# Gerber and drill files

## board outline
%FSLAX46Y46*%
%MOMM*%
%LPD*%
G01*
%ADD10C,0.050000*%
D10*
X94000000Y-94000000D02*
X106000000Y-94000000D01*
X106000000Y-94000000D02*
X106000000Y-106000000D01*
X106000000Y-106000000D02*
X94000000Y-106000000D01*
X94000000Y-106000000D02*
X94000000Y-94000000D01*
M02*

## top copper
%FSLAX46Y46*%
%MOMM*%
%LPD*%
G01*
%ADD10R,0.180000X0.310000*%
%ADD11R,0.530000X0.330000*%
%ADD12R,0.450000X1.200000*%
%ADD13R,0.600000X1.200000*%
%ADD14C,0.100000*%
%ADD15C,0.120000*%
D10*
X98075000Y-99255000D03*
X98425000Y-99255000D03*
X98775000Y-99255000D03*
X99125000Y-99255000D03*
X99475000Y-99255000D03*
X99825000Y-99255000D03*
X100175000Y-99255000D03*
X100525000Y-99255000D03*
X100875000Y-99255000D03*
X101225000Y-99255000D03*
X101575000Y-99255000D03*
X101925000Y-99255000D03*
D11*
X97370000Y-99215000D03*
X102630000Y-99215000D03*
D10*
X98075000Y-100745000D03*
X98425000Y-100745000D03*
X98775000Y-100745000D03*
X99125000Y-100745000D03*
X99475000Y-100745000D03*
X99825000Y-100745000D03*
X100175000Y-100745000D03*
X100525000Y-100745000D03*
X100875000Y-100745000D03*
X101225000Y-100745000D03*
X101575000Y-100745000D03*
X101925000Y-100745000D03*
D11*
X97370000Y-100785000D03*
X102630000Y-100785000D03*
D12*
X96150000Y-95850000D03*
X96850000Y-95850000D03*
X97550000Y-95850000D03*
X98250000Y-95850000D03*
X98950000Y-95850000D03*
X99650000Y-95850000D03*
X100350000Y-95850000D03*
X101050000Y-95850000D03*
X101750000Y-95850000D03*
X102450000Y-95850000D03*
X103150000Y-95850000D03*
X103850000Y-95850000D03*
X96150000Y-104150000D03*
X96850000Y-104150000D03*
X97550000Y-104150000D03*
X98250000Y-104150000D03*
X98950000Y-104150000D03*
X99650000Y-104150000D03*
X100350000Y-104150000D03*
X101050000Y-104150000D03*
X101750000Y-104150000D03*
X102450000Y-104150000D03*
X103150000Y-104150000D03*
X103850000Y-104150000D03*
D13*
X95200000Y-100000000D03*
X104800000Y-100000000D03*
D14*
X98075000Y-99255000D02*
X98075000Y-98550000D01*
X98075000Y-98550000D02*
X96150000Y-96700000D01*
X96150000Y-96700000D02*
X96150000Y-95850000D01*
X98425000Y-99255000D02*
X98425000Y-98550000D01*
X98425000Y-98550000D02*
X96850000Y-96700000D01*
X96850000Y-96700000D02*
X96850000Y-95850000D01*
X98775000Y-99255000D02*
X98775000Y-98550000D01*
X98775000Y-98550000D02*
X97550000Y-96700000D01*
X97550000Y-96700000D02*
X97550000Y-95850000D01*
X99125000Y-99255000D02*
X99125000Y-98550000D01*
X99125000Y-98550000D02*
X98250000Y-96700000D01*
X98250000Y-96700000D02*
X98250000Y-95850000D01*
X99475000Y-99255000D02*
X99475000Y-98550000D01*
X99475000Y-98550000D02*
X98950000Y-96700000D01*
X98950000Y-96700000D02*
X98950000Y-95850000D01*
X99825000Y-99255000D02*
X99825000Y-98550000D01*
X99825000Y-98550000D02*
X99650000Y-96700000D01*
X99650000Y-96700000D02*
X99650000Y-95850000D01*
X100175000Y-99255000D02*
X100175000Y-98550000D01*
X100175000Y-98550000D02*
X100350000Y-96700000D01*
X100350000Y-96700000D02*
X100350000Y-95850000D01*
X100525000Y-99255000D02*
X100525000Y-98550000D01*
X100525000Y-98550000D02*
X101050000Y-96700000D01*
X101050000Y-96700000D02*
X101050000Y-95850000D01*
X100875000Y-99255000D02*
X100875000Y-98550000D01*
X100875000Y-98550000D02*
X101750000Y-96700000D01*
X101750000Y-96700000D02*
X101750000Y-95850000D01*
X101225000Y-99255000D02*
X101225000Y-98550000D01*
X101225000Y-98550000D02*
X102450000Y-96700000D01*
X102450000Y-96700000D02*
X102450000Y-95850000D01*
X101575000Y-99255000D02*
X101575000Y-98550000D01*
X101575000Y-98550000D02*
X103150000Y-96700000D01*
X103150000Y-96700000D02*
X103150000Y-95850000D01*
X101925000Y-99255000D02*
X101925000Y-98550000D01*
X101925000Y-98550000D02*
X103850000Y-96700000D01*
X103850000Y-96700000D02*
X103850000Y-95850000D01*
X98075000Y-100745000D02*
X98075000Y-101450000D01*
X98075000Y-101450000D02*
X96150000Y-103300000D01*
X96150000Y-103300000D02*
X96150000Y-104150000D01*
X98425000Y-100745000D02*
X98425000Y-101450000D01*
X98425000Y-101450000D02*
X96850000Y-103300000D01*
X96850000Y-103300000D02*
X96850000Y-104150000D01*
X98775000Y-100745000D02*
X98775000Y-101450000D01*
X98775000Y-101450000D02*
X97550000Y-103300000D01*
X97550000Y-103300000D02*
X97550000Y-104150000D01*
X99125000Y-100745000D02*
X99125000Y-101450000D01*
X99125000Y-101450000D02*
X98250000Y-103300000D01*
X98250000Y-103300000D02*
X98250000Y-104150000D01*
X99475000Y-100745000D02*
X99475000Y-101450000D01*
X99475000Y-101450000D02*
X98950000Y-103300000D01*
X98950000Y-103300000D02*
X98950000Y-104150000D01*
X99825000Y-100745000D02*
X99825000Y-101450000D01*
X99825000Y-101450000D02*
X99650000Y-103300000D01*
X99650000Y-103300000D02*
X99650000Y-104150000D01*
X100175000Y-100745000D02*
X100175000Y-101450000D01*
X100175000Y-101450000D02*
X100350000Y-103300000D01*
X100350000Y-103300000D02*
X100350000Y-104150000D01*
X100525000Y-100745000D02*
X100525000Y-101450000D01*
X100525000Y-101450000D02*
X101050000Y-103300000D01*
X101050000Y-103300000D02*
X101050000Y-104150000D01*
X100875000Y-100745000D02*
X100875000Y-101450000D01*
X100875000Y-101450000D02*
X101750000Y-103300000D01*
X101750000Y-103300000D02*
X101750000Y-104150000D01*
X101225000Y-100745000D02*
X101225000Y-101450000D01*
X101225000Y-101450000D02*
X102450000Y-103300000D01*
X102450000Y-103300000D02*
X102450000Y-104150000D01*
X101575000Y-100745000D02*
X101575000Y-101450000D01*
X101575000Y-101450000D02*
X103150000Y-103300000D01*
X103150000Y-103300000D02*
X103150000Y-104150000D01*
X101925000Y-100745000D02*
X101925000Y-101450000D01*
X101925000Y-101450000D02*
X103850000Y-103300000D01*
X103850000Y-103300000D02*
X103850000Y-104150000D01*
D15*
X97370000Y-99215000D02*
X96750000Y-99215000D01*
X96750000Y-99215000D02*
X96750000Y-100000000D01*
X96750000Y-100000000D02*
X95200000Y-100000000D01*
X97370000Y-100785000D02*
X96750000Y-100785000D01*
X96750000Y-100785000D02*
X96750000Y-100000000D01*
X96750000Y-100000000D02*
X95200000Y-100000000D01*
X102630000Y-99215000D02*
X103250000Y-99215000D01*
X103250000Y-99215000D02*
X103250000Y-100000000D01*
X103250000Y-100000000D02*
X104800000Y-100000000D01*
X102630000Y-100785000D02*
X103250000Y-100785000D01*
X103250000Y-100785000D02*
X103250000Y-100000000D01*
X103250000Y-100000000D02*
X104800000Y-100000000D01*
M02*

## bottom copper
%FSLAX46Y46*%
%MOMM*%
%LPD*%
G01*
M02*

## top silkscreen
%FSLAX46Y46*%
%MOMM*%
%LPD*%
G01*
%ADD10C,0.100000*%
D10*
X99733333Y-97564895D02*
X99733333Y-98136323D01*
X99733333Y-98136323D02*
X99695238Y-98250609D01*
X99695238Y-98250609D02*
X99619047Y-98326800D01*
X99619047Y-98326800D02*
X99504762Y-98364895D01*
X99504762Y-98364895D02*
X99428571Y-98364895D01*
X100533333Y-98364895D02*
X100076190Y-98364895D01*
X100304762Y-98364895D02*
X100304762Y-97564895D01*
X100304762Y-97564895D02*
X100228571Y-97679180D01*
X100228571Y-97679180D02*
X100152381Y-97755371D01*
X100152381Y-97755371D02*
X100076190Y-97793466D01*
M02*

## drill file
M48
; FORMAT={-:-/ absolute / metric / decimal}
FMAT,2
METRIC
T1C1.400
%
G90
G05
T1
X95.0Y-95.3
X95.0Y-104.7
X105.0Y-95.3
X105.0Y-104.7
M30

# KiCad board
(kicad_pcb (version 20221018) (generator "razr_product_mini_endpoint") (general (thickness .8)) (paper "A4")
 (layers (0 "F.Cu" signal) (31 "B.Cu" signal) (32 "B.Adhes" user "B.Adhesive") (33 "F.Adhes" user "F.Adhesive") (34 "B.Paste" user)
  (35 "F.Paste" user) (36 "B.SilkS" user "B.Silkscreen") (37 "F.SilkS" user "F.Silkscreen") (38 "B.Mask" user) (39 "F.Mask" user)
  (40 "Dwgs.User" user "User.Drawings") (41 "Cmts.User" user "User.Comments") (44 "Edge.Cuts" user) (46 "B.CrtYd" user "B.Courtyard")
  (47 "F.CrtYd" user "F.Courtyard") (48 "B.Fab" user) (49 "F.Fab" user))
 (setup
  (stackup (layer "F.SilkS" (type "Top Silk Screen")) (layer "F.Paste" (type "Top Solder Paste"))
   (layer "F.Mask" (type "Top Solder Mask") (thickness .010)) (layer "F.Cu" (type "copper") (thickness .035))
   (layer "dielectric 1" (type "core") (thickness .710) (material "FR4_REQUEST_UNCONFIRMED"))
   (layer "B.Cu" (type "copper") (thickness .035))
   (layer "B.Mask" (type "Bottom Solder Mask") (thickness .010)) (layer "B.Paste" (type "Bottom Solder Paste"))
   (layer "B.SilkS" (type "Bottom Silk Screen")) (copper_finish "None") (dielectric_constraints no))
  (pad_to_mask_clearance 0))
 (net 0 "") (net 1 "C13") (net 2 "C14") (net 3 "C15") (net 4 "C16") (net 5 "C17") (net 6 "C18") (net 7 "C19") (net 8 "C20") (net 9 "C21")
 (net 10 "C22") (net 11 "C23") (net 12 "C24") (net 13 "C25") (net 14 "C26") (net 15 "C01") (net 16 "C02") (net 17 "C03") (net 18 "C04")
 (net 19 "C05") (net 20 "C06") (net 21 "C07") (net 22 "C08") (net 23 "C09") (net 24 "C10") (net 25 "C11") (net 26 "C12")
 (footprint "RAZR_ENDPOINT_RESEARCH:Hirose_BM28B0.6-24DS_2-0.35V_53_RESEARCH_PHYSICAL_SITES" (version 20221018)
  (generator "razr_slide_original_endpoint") (layer "F.Cu") (at 100 100)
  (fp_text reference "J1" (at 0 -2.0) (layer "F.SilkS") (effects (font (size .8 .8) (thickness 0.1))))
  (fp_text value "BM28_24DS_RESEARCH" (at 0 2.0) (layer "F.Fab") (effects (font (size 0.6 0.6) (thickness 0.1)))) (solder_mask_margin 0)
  (pad "S_NEG_00" smd rect (at -1.925 -0.745) (size 0.18 0.31) (layers "F.Cu" "F.Mask") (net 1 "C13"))
  (pad "S_NEG_01" smd rect (at -1.575 -0.745) (size 0.18 0.31) (layers "F.Cu" "F.Mask") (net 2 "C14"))
  (pad "S_NEG_02" smd rect (at -1.225 -0.745) (size 0.18 0.31) (layers "F.Cu" "F.Mask") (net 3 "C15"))
  (pad "S_NEG_03" smd rect (at -0.875 -0.745) (size 0.18 0.31) (layers "F.Cu" "F.Mask") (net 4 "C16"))
  (pad "S_NEG_04" smd rect (at -0.525 -0.745) (size 0.18 0.31) (layers "F.Cu" "F.Mask") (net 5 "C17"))
  (pad "S_NEG_05" smd rect (at -0.175 -0.745) (size 0.18 0.31) (layers "F.Cu" "F.Mask") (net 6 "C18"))
  (pad "S_NEG_06" smd rect (at 0.175 -0.745) (size 0.18 0.31) (layers "F.Cu" "F.Mask") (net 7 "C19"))
  (pad "S_NEG_07" smd rect (at 0.525 -0.745) (size 0.18 0.31) (layers "F.Cu" "F.Mask") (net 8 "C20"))
  (pad "S_NEG_08" smd rect (at 0.875 -0.745) (size 0.18 0.31) (layers "F.Cu" "F.Mask") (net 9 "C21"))
  (pad "S_NEG_09" smd rect (at 1.225 -0.745) (size 0.18 0.31) (layers "F.Cu" "F.Mask") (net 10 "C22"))
  (pad "S_NEG_10" smd rect (at 1.575 -0.745) (size 0.18 0.31) (layers "F.Cu" "F.Mask") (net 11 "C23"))
  (pad "S_NEG_11" smd rect (at 1.925 -0.745) (size 0.18 0.31) (layers "F.Cu" "F.Mask") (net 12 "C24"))
  (pad "P_L" smd rect (at -2.63 -0.785) (size 0.53 0.33) (layers "F.Cu" "F.Mask") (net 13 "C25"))
  (pad "P_R" smd rect (at 2.63 -0.785) (size 0.53 0.33) (layers "F.Cu" "F.Mask") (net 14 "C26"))
  (pad "S_POS_00" smd rect (at -1.925 0.745) (size 0.18 0.31) (layers "F.Cu" "F.Mask") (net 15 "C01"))
  (pad "S_POS_01" smd rect (at -1.575 0.745) (size 0.18 0.31) (layers "F.Cu" "F.Mask") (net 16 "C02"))
  (pad "S_POS_02" smd rect (at -1.225 0.745) (size 0.18 0.31) (layers "F.Cu" "F.Mask") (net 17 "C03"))
  (pad "S_POS_03" smd rect (at -0.875 0.745) (size 0.18 0.31) (layers "F.Cu" "F.Mask") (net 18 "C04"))
  (pad "S_POS_04" smd rect (at -0.525 0.745) (size 0.18 0.31) (layers "F.Cu" "F.Mask") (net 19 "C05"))
  (pad "S_POS_05" smd rect (at -0.175 0.745) (size 0.18 0.31) (layers "F.Cu" "F.Mask") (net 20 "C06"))
  (pad "S_POS_06" smd rect (at 0.175 0.745) (size 0.18 0.31) (layers "F.Cu" "F.Mask") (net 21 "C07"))
  (pad "S_POS_07" smd rect (at 0.525 0.745) (size 0.18 0.31) (layers "F.Cu" "F.Mask") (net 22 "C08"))
  (pad "S_POS_08" smd rect (at 0.875 0.745) (size 0.18 0.31) (layers "F.Cu" "F.Mask") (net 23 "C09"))
  (pad "S_POS_09" smd rect (at 1.225 0.745) (size 0.18 0.31) (layers "F.Cu" "F.Mask") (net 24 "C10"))
  (pad "S_POS_10" smd rect (at 1.575 0.745) (size 0.18 0.31) (layers "F.Cu" "F.Mask") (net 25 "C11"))
  (pad "S_POS_11" smd rect (at 1.925 0.745) (size 0.18 0.31) (layers "F.Cu" "F.Mask") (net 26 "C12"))
  (pad "P_L" smd rect (at -2.63 0.785) (size 0.53 0.33) (layers "F.Cu" "F.Mask") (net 13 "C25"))
  (pad "P_R" smd rect (at 2.63 0.785) (size 0.53 0.33) (layers "F.Cu" "F.Mask") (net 14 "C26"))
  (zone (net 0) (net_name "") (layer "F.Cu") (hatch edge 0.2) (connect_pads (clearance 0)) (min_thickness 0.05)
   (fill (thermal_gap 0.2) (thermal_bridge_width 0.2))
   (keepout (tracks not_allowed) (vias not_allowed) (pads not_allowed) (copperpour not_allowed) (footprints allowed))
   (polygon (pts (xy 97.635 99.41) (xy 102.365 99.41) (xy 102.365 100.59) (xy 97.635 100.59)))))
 (segment (start 98.075000 99.255000) (end 98.075000 98.550000) (width 0.1) (layer "F.Cu") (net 1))
 (segment (start 98.075000 98.550000) (end 96.150000 96.700000) (width 0.1) (layer "F.Cu") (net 1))
 (segment (start 96.150000 96.700000) (end 96.150000 95.850000) (width 0.1) (layer "F.Cu") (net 1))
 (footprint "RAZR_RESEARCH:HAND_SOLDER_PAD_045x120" (layer "F.Cu") (at 96.150000 95.850000)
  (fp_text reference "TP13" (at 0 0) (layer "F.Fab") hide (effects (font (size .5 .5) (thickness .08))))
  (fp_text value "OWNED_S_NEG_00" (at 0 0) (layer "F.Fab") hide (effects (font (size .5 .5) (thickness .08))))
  (pad "1" smd rect (at 0 0) (size 0.45 1.2) (layers "F.Cu" "F.Mask") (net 1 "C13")))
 (segment (start 98.425000 99.255000) (end 98.425000 98.550000) (width 0.1) (layer "F.Cu") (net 2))
 (segment (start 98.425000 98.550000) (end 96.850000 96.700000) (width 0.1) (layer "F.Cu") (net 2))
 (segment (start 96.850000 96.700000) (end 96.850000 95.850000) (width 0.1) (layer "F.Cu") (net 2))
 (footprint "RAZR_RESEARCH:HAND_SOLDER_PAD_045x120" (layer "F.Cu") (at 96.850000 95.850000)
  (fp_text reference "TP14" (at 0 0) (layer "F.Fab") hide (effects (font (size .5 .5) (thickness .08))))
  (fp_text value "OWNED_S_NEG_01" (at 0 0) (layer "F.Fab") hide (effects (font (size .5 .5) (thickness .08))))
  (pad "1" smd rect (at 0 0) (size 0.45 1.2) (layers "F.Cu" "F.Mask") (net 2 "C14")))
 (segment (start 98.775000 99.255000) (end 98.775000 98.550000) (width 0.1) (layer "F.Cu") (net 3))
 (segment (start 98.775000 98.550000) (end 97.550000 96.700000) (width 0.1) (layer "F.Cu") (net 3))
 (segment (start 97.550000 96.700000) (end 97.550000 95.850000) (width 0.1) (layer "F.Cu") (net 3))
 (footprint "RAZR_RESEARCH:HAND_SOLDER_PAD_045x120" (layer "F.Cu") (at 97.550000 95.850000)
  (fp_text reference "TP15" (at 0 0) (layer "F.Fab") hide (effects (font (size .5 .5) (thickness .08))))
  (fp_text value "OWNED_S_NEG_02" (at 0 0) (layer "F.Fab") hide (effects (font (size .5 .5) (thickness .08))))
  (pad "1" smd rect (at 0 0) (size 0.45 1.2) (layers "F.Cu" "F.Mask") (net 3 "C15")))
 (segment (start 99.125000 99.255000) (end 99.125000 98.550000) (width 0.1) (layer "F.Cu") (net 4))
 (segment (start 99.125000 98.550000) (end 98.250000 96.700000) (width 0.1) (layer "F.Cu") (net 4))
 (segment (start 98.250000 96.700000) (end 98.250000 95.850000) (width 0.1) (layer "F.Cu") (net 4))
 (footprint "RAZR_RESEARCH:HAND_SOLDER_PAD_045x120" (layer "F.Cu") (at 98.250000 95.850000)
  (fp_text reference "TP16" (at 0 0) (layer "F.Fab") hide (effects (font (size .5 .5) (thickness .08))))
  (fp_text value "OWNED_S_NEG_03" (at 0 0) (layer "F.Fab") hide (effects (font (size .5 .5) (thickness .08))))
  (pad "1" smd rect (at 0 0) (size 0.45 1.2) (layers "F.Cu" "F.Mask") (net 4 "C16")))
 (segment (start 99.475000 99.255000) (end 99.475000 98.550000) (width 0.1) (layer "F.Cu") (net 5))
 (segment (start 99.475000 98.550000) (end 98.950000 96.700000) (width 0.1) (layer "F.Cu") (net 5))
 (segment (start 98.950000 96.700000) (end 98.950000 95.850000) (width 0.1) (layer "F.Cu") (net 5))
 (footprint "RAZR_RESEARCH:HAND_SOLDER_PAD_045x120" (layer "F.Cu") (at 98.950000 95.850000)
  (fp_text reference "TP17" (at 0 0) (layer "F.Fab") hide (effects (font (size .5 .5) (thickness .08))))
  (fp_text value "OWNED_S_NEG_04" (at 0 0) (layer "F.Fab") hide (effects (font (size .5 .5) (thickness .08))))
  (pad "1" smd rect (at 0 0) (size 0.45 1.2) (layers "F.Cu" "F.Mask") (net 5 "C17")))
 (segment (start 99.825000 99.255000) (end 99.825000 98.550000) (width 0.1) (layer "F.Cu") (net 6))
 (segment (start 99.825000 98.550000) (end 99.650000 96.700000) (width 0.1) (layer "F.Cu") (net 6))
 (segment (start 99.650000 96.700000) (end 99.650000 95.850000) (width 0.1) (layer "F.Cu") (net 6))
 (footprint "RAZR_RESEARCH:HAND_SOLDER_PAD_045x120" (layer "F.Cu") (at 99.650000 95.850000)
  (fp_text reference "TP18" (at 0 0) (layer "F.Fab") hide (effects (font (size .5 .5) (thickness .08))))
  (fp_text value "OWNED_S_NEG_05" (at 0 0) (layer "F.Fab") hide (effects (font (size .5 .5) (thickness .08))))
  (pad "1" smd rect (at 0 0) (size 0.45 1.2) (layers "F.Cu" "F.Mask") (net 6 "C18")))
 (segment (start 100.175000 99.255000) (end 100.175000 98.550000) (width 0.1) (layer "F.Cu") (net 7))
 (segment (start 100.175000 98.550000) (end 100.350000 96.700000) (width 0.1) (layer "F.Cu") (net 7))
 (segment (start 100.350000 96.700000) (end 100.350000 95.850000) (width 0.1) (layer "F.Cu") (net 7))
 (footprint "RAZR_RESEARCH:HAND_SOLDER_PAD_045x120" (layer "F.Cu") (at 100.350000 95.850000)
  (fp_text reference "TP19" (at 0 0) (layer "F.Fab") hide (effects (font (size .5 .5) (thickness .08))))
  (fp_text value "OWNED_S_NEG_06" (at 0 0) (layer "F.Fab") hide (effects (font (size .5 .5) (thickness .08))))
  (pad "1" smd rect (at 0 0) (size 0.45 1.2) (layers "F.Cu" "F.Mask") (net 7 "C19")))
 (segment (start 100.525000 99.255000) (end 100.525000 98.550000) (width 0.1) (layer "F.Cu") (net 8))
 (segment (start 100.525000 98.550000) (end 101.050000 96.700000) (width 0.1) (layer "F.Cu") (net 8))
 (segment (start 101.050000 96.700000) (end 101.050000 95.850000) (width 0.1) (layer "F.Cu") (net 8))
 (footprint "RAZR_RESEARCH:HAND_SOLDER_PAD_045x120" (layer "F.Cu") (at 101.050000 95.850000)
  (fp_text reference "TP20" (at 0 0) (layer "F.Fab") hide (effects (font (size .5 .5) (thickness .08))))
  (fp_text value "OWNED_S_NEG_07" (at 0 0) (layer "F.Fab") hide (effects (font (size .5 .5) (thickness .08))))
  (pad "1" smd rect (at 0 0) (size 0.45 1.2) (layers "F.Cu" "F.Mask") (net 8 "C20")))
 (segment (start 100.875000 99.255000) (end 100.875000 98.550000) (width 0.1) (layer "F.Cu") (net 9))
 (segment (start 100.875000 98.550000) (end 101.750000 96.700000) (width 0.1) (layer "F.Cu") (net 9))
 (segment (start 101.750000 96.700000) (end 101.750000 95.850000) (width 0.1) (layer "F.Cu") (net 9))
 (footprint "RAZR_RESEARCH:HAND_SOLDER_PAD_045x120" (layer "F.Cu") (at 101.750000 95.850000)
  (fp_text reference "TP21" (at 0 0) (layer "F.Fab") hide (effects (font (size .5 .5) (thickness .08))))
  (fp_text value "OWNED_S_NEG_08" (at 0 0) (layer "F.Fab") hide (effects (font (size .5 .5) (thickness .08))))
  (pad "1" smd rect (at 0 0) (size 0.45 1.2) (layers "F.Cu" "F.Mask") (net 9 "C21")))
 (segment (start 101.225000 99.255000) (end 101.225000 98.550000) (width 0.1) (layer "F.Cu") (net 10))
 (segment (start 101.225000 98.550000) (end 102.450000 96.700000) (width 0.1) (layer "F.Cu") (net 10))
 (segment (start 102.450000 96.700000) (end 102.450000 95.850000) (width 0.1) (layer "F.Cu") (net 10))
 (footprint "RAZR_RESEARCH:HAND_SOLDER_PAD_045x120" (layer "F.Cu") (at 102.450000 95.850000)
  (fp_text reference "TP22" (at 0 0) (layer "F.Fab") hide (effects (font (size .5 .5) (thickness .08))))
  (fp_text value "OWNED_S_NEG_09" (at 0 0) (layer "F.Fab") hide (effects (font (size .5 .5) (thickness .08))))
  (pad "1" smd rect (at 0 0) (size 0.45 1.2) (layers "F.Cu" "F.Mask") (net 10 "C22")))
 (segment (start 101.575000 99.255000) (end 101.575000 98.550000) (width 0.1) (layer "F.Cu") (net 11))
 (segment (start 101.575000 98.550000) (end 103.150000 96.700000) (width 0.1) (layer "F.Cu") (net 11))
 (segment (start 103.150000 96.700000) (end 103.150000 95.850000) (width 0.1) (layer "F.Cu") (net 11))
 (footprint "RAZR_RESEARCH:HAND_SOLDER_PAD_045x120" (layer "F.Cu") (at 103.150000 95.850000)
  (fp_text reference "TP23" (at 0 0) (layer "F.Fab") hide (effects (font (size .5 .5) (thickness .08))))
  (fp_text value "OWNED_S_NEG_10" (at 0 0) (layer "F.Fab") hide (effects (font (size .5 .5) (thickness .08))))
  (pad "1" smd rect (at 0 0) (size 0.45 1.2) (layers "F.Cu" "F.Mask") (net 11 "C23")))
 (segment (start 101.925000 99.255000) (end 101.925000 98.550000) (width 0.1) (layer "F.Cu") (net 12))
 (segment (start 101.925000 98.550000) (end 103.850000 96.700000) (width 0.1) (layer "F.Cu") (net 12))
 (segment (start 103.850000 96.700000) (end 103.850000 95.850000) (width 0.1) (layer "F.Cu") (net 12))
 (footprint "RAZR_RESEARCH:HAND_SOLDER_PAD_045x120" (layer "F.Cu") (at 103.850000 95.850000)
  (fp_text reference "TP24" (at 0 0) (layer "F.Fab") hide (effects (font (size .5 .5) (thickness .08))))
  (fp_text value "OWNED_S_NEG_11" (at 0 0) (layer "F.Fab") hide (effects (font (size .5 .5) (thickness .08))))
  (pad "1" smd rect (at 0 0) (size 0.45 1.2) (layers "F.Cu" "F.Mask") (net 12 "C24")))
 (segment (start 98.075000 100.745000) (end 98.075000 101.450000) (width 0.1) (layer "F.Cu") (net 15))
 (segment (start 98.075000 101.450000) (end 96.150000 103.300000) (width 0.1) (layer "F.Cu") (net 15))
 (segment (start 96.150000 103.300000) (end 96.150000 104.150000) (width 0.1) (layer "F.Cu") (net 15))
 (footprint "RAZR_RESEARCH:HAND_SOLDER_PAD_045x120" (layer "F.Cu") (at 96.150000 104.150000)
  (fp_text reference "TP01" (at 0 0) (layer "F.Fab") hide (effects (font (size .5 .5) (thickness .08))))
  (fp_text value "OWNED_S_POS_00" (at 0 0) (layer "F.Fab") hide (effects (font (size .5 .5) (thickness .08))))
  (pad "1" smd rect (at 0 0) (size 0.45 1.2) (layers "F.Cu" "F.Mask") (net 15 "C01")))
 (segment (start 98.425000 100.745000) (end 98.425000 101.450000) (width 0.1) (layer "F.Cu") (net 16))
 (segment (start 98.425000 101.450000) (end 96.850000 103.300000) (width 0.1) (layer "F.Cu") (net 16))
 (segment (start 96.850000 103.300000) (end 96.850000 104.150000) (width 0.1) (layer "F.Cu") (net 16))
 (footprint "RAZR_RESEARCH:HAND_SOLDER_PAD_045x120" (layer "F.Cu") (at 96.850000 104.150000)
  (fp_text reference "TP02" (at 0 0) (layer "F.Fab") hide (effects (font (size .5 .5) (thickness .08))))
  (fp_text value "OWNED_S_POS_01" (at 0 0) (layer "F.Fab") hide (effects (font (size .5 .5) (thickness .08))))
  (pad "1" smd rect (at 0 0) (size 0.45 1.2) (layers "F.Cu" "F.Mask") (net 16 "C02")))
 (segment (start 98.775000 100.745000) (end 98.775000 101.450000) (width 0.1) (layer "F.Cu") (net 17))
 (segment (start 98.775000 101.450000) (end 97.550000 103.300000) (width 0.1) (layer "F.Cu") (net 17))
 (segment (start 97.550000 103.300000) (end 97.550000 104.150000) (width 0.1) (layer "F.Cu") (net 17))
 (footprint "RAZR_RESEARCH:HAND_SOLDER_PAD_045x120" (layer "F.Cu") (at 97.550000 104.150000)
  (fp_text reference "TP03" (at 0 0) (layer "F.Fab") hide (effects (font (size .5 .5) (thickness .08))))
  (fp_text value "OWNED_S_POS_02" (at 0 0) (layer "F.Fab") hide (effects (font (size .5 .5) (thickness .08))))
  (pad "1" smd rect (at 0 0) (size 0.45 1.2) (layers "F.Cu" "F.Mask") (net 17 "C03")))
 (segment (start 99.125000 100.745000) (end 99.125000 101.450000) (width 0.1) (layer "F.Cu") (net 18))
 (segment (start 99.125000 101.450000) (end 98.250000 103.300000) (width 0.1) (layer "F.Cu") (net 18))
 (segment (start 98.250000 103.300000) (end 98.250000 104.150000) (width 0.1) (layer "F.Cu") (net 18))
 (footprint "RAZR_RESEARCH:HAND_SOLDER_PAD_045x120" (layer "F.Cu") (at 98.250000 104.150000)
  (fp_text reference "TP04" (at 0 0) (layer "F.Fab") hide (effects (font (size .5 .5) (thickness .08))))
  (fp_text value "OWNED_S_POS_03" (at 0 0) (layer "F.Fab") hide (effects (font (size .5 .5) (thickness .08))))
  (pad "1" smd rect (at 0 0) (size 0.45 1.2) (layers "F.Cu" "F.Mask") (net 18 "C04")))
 (segment (start 99.475000 100.745000) (end 99.475000 101.450000) (width 0.1) (layer "F.Cu") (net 19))
 (segment (start 99.475000 101.450000) (end 98.950000 103.300000) (width 0.1) (layer "F.Cu") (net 19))
 (segment (start 98.950000 103.300000) (end 98.950000 104.150000) (width 0.1) (layer "F.Cu") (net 19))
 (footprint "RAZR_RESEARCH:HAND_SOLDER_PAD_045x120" (layer "F.Cu") (at 98.950000 104.150000)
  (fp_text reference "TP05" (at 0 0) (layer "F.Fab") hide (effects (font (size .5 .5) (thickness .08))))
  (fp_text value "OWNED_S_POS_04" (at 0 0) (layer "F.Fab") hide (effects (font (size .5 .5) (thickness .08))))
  (pad "1" smd rect (at 0 0) (size 0.45 1.2) (layers "F.Cu" "F.Mask") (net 19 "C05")))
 (segment (start 99.825000 100.745000) (end 99.825000 101.450000) (width 0.1) (layer "F.Cu") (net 20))
 (segment (start 99.825000 101.450000) (end 99.650000 103.300000) (width 0.1) (layer "F.Cu") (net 20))
 (segment (start 99.650000 103.300000) (end 99.650000 104.150000) (width 0.1) (layer "F.Cu") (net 20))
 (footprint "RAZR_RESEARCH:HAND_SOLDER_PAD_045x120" (layer "F.Cu") (at 99.650000 104.150000)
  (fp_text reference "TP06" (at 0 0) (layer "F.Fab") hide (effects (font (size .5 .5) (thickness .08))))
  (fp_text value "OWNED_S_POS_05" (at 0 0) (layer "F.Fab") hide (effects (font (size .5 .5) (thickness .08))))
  (pad "1" smd rect (at 0 0) (size 0.45 1.2) (layers "F.Cu" "F.Mask") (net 20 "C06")))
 (segment (start 100.175000 100.745000) (end 100.175000 101.450000) (width 0.1) (layer "F.Cu") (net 21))
 (segment (start 100.175000 101.450000) (end 100.350000 103.300000) (width 0.1) (layer "F.Cu") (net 21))
 (segment (start 100.350000 103.300000) (end 100.350000 104.150000) (width 0.1) (layer "F.Cu") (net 21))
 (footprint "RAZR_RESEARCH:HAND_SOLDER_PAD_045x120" (layer "F.Cu") (at 100.350000 104.150000)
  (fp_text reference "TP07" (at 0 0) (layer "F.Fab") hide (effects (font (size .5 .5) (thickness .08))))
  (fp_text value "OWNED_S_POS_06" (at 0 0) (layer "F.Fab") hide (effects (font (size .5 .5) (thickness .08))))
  (pad "1" smd rect (at 0 0) (size 0.45 1.2) (layers "F.Cu" "F.Mask") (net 21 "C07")))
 (segment (start 100.525000 100.745000) (end 100.525000 101.450000) (width 0.1) (layer "F.Cu") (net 22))
 (segment (start 100.525000 101.450000) (end 101.050000 103.300000) (width 0.1) (layer "F.Cu") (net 22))
 (segment (start 101.050000 103.300000) (end 101.050000 104.150000) (width 0.1) (layer "F.Cu") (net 22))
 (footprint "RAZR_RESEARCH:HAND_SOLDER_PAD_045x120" (layer "F.Cu") (at 101.050000 104.150000)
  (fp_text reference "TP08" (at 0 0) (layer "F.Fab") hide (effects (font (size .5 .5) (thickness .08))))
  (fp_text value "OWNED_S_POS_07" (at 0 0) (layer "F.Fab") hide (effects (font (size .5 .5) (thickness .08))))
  (pad "1" smd rect (at 0 0) (size 0.45 1.2) (layers "F.Cu" "F.Mask") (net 22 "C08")))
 (segment (start 100.875000 100.745000) (end 100.875000 101.450000) (width 0.1) (layer "F.Cu") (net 23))
 (segment (start 100.875000 101.450000) (end 101.750000 103.300000) (width 0.1) (layer "F.Cu") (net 23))
 (segment (start 101.750000 103.300000) (end 101.750000 104.150000) (width 0.1) (layer "F.Cu") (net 23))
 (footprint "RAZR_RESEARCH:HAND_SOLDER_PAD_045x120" (layer "F.Cu") (at 101.750000 104.150000)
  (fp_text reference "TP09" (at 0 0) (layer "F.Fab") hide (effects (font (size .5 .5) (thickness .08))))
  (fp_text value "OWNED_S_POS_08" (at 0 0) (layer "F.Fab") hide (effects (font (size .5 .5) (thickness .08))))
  (pad "1" smd rect (at 0 0) (size 0.45 1.2) (layers "F.Cu" "F.Mask") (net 23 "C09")))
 (segment (start 101.225000 100.745000) (end 101.225000 101.450000) (width 0.1) (layer "F.Cu") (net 24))
 (segment (start 101.225000 101.450000) (end 102.450000 103.300000) (width 0.1) (layer "F.Cu") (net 24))
 (segment (start 102.450000 103.300000) (end 102.450000 104.150000) (width 0.1) (layer "F.Cu") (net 24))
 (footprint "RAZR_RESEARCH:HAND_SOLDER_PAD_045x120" (layer "F.Cu") (at 102.450000 104.150000)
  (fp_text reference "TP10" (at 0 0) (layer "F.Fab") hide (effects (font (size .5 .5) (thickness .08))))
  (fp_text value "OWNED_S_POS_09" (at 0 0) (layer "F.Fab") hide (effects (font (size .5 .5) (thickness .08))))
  (pad "1" smd rect (at 0 0) (size 0.45 1.2) (layers "F.Cu" "F.Mask") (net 24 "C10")))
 (segment (start 101.575000 100.745000) (end 101.575000 101.450000) (width 0.1) (layer "F.Cu") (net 25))
 (segment (start 101.575000 101.450000) (end 103.150000 103.300000) (width 0.1) (layer "F.Cu") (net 25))
 (segment (start 103.150000 103.300000) (end 103.150000 104.150000) (width 0.1) (layer "F.Cu") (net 25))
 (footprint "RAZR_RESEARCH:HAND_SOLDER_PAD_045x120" (layer "F.Cu") (at 103.150000 104.150000)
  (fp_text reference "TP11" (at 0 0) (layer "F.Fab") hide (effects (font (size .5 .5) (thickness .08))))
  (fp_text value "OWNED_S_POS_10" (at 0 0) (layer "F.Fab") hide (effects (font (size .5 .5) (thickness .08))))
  (pad "1" smd rect (at 0 0) (size 0.45 1.2) (layers "F.Cu" "F.Mask") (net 25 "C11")))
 (segment (start 101.925000 100.745000) (end 101.925000 101.450000) (width 0.1) (layer "F.Cu") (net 26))
 (segment (start 101.925000 101.450000) (end 103.850000 103.300000) (width 0.1) (layer "F.Cu") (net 26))
 (segment (start 103.850000 103.300000) (end 103.850000 104.150000) (width 0.1) (layer "F.Cu") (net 26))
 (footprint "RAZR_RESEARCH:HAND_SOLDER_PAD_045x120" (layer "F.Cu") (at 103.850000 104.150000)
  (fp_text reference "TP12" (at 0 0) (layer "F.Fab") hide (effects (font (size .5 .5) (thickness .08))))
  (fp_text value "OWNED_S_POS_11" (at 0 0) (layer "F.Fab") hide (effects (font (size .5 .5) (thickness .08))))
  (pad "1" smd rect (at 0 0) (size 0.45 1.2) (layers "F.Cu" "F.Mask") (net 26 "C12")))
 (segment (start 97.370000 99.215000) (end 96.750000 99.215000) (width 0.12) (layer "F.Cu") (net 13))
 (segment (start 96.750000 99.215000) (end 96.750000 100.000000) (width 0.12) (layer "F.Cu") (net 13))
 (segment (start 96.750000 100.000000) (end 95.200000 100.000000) (width 0.12) (layer "F.Cu") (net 13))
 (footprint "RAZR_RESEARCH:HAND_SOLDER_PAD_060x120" (layer "F.Cu") (at 95.200000 100.000000)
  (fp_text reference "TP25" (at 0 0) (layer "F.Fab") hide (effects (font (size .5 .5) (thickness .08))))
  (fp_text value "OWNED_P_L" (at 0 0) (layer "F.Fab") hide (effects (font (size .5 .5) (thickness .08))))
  (pad "1" smd rect (at 0 0) (size 0.6 1.2) (layers "F.Cu" "F.Mask") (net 13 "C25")))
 (segment (start 97.370000 100.785000) (end 96.750000 100.785000) (width 0.12) (layer "F.Cu") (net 13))
 (segment (start 96.750000 100.785000) (end 96.750000 100.000000) (width 0.12) (layer "F.Cu") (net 13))
 (segment (start 96.750000 100.000000) (end 95.200000 100.000000) (width 0.12) (layer "F.Cu") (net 13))
 (segment (start 102.630000 99.215000) (end 103.250000 99.215000) (width 0.12) (layer "F.Cu") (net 14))
 (segment (start 103.250000 99.215000) (end 103.250000 100.000000) (width 0.12) (layer "F.Cu") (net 14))
 (segment (start 103.250000 100.000000) (end 104.800000 100.000000) (width 0.12) (layer "F.Cu") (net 14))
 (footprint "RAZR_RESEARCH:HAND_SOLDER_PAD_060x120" (layer "F.Cu") (at 104.800000 100.000000)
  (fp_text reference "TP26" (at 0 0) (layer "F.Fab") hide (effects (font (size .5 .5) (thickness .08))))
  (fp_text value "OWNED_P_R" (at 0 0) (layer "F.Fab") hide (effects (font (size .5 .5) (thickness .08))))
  (pad "1" smd rect (at 0 0) (size 0.6 1.2) (layers "F.Cu" "F.Mask") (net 14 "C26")))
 (segment (start 102.630000 100.785000) (end 103.250000 100.785000) (width 0.12) (layer "F.Cu") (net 14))
 (segment (start 103.250000 100.785000) (end 103.250000 100.000000) (width 0.12) (layer "F.Cu") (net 14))
 (segment (start 103.250000 100.000000) (end 104.800000 100.000000) (width 0.12) (layer "F.Cu") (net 14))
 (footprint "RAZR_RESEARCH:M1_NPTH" (layer "F.Cu") (at 95 95.3)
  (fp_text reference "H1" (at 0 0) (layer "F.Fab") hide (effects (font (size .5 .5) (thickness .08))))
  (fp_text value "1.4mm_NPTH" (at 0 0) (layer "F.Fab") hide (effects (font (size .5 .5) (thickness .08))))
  (pad "" np_thru_hole circle (at 0 0) (size 1.4 1.4) (drill 1.4) (layers "*.Cu" "*.Mask")))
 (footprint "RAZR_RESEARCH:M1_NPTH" (layer "F.Cu") (at 105 95.3)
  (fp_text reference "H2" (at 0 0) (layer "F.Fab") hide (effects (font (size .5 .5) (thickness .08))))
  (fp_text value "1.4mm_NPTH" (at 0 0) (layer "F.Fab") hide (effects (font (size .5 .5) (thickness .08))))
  (pad "" np_thru_hole circle (at 0 0) (size 1.4 1.4) (drill 1.4) (layers "*.Cu" "*.Mask")))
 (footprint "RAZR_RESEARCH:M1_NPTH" (layer "F.Cu") (at 95 104.7)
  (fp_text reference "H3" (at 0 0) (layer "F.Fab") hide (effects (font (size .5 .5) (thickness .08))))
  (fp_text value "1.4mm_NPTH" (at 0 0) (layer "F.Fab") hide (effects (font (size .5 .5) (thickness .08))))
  (pad "" np_thru_hole circle (at 0 0) (size 1.4 1.4) (drill 1.4) (layers "*.Cu" "*.Mask")))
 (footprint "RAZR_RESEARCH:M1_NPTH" (layer "F.Cu") (at 105 104.7)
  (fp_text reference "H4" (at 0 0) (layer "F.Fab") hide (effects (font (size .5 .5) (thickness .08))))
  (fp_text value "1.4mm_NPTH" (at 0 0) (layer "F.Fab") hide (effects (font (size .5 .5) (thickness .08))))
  (pad "" np_thru_hole circle (at 0 0) (size 1.4 1.4) (drill 1.4) (layers "*.Cu" "*.Mask")))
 (gr_line (start 94 94) (end 106 94) (layer "Edge.Cuts") (width .05))
 (gr_line (start 106 94) (end 106 106) (layer "Edge.Cuts") (width .05))
 (gr_line (start 106 106) (end 94 106) (layer "Edge.Cuts") (width .05))
 (gr_line (start 94 106) (end 94 94) (layer "Edge.Cuts") (width .05)))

